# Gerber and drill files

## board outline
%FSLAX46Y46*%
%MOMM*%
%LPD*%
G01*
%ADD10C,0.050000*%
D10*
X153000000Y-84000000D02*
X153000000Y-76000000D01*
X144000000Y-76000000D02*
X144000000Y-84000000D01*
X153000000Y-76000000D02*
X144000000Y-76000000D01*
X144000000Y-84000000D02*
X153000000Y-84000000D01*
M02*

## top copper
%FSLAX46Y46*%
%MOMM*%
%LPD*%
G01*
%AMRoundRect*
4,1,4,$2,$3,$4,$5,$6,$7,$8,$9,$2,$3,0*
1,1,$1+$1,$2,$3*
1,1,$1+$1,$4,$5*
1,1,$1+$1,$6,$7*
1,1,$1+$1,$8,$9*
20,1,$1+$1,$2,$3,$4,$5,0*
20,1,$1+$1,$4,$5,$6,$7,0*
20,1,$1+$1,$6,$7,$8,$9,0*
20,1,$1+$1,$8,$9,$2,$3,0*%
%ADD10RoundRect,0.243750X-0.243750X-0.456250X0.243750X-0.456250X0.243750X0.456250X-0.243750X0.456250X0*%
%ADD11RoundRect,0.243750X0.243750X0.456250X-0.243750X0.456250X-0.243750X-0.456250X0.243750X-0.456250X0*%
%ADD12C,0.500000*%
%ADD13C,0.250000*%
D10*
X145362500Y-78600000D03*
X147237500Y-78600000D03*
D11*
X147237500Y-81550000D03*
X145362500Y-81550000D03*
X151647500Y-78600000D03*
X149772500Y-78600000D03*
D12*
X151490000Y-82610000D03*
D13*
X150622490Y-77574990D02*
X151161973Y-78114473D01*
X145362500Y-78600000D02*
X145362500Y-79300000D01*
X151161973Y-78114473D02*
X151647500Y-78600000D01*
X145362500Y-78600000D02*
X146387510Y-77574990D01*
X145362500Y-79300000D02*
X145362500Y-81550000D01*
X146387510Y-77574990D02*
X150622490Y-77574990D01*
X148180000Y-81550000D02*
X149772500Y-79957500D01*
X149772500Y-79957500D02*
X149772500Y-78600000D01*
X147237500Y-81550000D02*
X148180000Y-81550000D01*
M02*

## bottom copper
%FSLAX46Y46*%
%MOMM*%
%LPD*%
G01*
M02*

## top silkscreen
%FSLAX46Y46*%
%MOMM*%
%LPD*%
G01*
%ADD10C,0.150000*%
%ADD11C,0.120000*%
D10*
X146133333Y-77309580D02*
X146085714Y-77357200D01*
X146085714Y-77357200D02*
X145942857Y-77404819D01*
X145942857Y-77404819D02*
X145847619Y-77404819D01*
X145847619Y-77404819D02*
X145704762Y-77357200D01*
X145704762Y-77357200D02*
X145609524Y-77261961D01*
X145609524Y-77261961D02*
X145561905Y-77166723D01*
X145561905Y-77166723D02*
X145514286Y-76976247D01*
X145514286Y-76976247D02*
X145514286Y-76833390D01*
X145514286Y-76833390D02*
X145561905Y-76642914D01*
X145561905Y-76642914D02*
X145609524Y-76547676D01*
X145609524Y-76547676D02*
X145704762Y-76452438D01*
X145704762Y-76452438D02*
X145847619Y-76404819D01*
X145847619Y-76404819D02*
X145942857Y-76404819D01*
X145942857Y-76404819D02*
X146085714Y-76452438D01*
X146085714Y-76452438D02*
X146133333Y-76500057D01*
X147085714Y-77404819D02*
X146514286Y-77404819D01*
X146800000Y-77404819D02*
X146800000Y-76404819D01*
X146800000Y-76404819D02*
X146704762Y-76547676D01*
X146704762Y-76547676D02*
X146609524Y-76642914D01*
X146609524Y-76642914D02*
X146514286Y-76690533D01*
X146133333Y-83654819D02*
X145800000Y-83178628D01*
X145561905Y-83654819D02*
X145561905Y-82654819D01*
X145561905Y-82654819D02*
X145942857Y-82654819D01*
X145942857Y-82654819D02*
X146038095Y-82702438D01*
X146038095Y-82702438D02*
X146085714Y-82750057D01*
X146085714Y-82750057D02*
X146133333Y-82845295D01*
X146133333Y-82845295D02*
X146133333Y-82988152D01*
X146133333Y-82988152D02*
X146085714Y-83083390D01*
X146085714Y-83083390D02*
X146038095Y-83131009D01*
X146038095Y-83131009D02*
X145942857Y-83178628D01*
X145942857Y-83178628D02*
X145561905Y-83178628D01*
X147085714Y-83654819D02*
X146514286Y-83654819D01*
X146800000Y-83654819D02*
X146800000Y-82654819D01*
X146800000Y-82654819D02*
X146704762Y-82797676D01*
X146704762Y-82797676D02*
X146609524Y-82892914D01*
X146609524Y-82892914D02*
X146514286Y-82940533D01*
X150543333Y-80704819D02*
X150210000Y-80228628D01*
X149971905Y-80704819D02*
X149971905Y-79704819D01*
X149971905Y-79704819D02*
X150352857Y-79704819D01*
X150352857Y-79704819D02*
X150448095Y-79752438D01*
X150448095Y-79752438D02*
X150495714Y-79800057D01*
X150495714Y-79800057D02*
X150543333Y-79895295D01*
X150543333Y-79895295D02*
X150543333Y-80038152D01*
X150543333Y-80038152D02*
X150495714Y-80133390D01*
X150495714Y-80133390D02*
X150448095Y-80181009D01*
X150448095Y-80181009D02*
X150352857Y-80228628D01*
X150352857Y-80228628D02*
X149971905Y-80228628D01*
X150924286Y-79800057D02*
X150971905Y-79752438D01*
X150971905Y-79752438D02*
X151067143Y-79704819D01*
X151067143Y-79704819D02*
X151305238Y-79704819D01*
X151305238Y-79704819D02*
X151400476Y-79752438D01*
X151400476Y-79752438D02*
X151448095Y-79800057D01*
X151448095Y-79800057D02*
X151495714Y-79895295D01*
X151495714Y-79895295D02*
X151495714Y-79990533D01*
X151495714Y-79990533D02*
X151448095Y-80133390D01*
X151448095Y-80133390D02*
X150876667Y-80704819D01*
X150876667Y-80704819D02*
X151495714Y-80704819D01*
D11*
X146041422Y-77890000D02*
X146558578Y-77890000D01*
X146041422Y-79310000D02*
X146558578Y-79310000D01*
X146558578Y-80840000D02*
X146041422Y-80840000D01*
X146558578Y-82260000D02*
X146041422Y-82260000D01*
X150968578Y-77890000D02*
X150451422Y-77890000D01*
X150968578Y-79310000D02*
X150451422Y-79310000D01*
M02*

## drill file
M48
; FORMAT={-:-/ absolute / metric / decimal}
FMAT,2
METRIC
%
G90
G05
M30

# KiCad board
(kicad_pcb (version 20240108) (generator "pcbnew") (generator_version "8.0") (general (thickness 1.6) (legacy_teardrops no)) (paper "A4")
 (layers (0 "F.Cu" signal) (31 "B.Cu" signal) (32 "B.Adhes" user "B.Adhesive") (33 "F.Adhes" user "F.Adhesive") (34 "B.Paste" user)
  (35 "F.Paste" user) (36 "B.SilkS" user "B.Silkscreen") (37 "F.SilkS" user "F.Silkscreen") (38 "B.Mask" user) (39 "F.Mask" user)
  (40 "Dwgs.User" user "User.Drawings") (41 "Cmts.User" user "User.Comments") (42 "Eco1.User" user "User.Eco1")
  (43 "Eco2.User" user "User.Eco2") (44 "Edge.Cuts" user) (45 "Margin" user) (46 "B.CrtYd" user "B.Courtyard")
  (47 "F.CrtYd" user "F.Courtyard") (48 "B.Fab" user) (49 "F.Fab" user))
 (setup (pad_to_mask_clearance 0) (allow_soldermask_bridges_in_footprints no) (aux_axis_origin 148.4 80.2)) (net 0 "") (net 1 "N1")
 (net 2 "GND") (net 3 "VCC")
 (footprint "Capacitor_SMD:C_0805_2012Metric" (layer "F.Cu") (at 146.3 78.6)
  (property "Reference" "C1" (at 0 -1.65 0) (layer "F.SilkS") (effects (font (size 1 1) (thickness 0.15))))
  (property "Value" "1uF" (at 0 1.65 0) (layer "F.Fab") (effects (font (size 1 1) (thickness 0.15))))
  (fp_line (start -0.258578 -0.71) (end 0.258578 -0.71) (stroke (width 0.12) (type solid)) (layer "F.SilkS"))
  (fp_line (start -0.258578 0.71) (end 0.258578 0.71) (stroke (width 0.12) (type solid)) (layer "F.SilkS"))
  (pad "1" smd roundrect (at -0.9375 0) (size 0.975 1.4) (layers "F.Cu" "F.Paste" "F.Mask") (roundrect_rratio 0.25) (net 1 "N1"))
  (pad "2" smd roundrect (at 0.9375 0) (size 0.975 1.4) (layers "F.Cu" "F.Paste" "F.Mask") (roundrect_rratio 0.25) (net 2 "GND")))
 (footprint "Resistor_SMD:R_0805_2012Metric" (layer "F.Cu") (at 146.3 81.55 180)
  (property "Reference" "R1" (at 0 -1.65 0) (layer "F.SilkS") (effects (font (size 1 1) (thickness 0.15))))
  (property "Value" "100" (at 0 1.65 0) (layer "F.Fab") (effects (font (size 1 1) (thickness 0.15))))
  (fp_line (start -0.258578 0.71) (end 0.258578 0.71) (stroke (width 0.12) (type solid)) (layer "F.SilkS"))
  (fp_line (start -0.258578 -0.71) (end 0.258578 -0.71) (stroke (width 0.12) (type solid)) (layer "F.SilkS"))
  (pad "1" smd roundrect (at -0.9375 0 180) (size 0.975 1.4) (layers "F.Cu" "F.Paste" "F.Mask") (roundrect_rratio 0.25) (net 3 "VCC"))
  (pad "2" smd roundrect (at 0.9375 0 180) (size 0.975 1.4) (layers "F.Cu" "F.Paste" "F.Mask") (roundrect_rratio 0.25) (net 1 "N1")))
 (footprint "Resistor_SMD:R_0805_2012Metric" (layer "F.Cu") (at 150.71 78.6 180)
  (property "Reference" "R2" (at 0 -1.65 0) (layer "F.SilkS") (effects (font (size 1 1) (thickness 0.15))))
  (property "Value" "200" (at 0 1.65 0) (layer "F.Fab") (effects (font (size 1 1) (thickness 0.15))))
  (fp_line (start -0.258578 0.71) (end 0.258578 0.71) (stroke (width 0.12) (type solid)) (layer "F.SilkS"))
  (fp_line (start -0.258578 -0.71) (end 0.258578 -0.71) (stroke (width 0.12) (type solid)) (layer "F.SilkS"))
  (pad "1" smd roundrect (at -0.9375 0 180) (size 0.975 1.4) (layers "F.Cu" "F.Paste" "F.Mask") (roundrect_rratio 0.25) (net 1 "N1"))
  (pad "2" smd roundrect (at 0.9375 0 180) (size 0.975 1.4) (layers "F.Cu" "F.Paste" "F.Mask") (roundrect_rratio 0.25) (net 3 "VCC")))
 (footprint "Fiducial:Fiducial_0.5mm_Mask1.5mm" (layer "F.Cu") (at 151.49 82.61)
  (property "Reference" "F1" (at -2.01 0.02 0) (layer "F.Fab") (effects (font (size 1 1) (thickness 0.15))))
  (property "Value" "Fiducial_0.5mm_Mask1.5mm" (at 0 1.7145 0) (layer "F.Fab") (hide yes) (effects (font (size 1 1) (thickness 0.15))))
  (pad "" smd circle (at 0 0) (size 0.5 0.5) (layers "F.Cu" "F.Mask") (solder_mask_margin 0.5) (clearance 0.5)))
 (gr_line (start 153 84) (end 153 76) (stroke (width 0.05) (type solid)) (layer "Edge.Cuts"))
 (gr_line (start 144 76) (end 144 84) (stroke (width 0.05) (type solid)) (layer "Edge.Cuts"))
 (gr_line (start 153 76) (end 144 76) (stroke (width 0.05) (type solid)) (layer "Edge.Cuts"))
 (gr_line (start 144 84) (end 153 84) (stroke (width 0.05) (type solid)) (layer "Edge.Cuts"))
 (segment (start 150.62249 77.57499) (end 151.161973 78.114473) (width 0.25) (layer "F.Cu") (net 1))
 (segment (start 145.3625 78.6) (end 145.3625 79.3) (width 0.25) (layer "F.Cu") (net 1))
 (segment (start 151.161973 78.114473) (end 151.6475 78.6) (width 0.25) (layer "F.Cu") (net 1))
 (segment (start 145.3625 78.6) (end 146.38751 77.57499) (width 0.25) (layer "F.Cu") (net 1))
 (segment (start 145.3625 79.3) (end 145.3625 81.55) (width 0.25) (layer "F.Cu") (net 1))
 (segment (start 146.38751 77.57499) (end 150.62249 77.57499) (width 0.25) (layer "F.Cu") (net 1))
 (segment (start 148.18 81.55) (end 149.7725 79.9575) (width 0.25) (layer "F.Cu") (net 3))
 (segment (start 149.7725 79.9575) (end 149.7725 78.6) (width 0.25) (layer "F.Cu") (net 3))
 (segment (start 147.2375 81.55) (end 148.18 81.55) (width 0.25) (layer "F.Cu") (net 3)))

